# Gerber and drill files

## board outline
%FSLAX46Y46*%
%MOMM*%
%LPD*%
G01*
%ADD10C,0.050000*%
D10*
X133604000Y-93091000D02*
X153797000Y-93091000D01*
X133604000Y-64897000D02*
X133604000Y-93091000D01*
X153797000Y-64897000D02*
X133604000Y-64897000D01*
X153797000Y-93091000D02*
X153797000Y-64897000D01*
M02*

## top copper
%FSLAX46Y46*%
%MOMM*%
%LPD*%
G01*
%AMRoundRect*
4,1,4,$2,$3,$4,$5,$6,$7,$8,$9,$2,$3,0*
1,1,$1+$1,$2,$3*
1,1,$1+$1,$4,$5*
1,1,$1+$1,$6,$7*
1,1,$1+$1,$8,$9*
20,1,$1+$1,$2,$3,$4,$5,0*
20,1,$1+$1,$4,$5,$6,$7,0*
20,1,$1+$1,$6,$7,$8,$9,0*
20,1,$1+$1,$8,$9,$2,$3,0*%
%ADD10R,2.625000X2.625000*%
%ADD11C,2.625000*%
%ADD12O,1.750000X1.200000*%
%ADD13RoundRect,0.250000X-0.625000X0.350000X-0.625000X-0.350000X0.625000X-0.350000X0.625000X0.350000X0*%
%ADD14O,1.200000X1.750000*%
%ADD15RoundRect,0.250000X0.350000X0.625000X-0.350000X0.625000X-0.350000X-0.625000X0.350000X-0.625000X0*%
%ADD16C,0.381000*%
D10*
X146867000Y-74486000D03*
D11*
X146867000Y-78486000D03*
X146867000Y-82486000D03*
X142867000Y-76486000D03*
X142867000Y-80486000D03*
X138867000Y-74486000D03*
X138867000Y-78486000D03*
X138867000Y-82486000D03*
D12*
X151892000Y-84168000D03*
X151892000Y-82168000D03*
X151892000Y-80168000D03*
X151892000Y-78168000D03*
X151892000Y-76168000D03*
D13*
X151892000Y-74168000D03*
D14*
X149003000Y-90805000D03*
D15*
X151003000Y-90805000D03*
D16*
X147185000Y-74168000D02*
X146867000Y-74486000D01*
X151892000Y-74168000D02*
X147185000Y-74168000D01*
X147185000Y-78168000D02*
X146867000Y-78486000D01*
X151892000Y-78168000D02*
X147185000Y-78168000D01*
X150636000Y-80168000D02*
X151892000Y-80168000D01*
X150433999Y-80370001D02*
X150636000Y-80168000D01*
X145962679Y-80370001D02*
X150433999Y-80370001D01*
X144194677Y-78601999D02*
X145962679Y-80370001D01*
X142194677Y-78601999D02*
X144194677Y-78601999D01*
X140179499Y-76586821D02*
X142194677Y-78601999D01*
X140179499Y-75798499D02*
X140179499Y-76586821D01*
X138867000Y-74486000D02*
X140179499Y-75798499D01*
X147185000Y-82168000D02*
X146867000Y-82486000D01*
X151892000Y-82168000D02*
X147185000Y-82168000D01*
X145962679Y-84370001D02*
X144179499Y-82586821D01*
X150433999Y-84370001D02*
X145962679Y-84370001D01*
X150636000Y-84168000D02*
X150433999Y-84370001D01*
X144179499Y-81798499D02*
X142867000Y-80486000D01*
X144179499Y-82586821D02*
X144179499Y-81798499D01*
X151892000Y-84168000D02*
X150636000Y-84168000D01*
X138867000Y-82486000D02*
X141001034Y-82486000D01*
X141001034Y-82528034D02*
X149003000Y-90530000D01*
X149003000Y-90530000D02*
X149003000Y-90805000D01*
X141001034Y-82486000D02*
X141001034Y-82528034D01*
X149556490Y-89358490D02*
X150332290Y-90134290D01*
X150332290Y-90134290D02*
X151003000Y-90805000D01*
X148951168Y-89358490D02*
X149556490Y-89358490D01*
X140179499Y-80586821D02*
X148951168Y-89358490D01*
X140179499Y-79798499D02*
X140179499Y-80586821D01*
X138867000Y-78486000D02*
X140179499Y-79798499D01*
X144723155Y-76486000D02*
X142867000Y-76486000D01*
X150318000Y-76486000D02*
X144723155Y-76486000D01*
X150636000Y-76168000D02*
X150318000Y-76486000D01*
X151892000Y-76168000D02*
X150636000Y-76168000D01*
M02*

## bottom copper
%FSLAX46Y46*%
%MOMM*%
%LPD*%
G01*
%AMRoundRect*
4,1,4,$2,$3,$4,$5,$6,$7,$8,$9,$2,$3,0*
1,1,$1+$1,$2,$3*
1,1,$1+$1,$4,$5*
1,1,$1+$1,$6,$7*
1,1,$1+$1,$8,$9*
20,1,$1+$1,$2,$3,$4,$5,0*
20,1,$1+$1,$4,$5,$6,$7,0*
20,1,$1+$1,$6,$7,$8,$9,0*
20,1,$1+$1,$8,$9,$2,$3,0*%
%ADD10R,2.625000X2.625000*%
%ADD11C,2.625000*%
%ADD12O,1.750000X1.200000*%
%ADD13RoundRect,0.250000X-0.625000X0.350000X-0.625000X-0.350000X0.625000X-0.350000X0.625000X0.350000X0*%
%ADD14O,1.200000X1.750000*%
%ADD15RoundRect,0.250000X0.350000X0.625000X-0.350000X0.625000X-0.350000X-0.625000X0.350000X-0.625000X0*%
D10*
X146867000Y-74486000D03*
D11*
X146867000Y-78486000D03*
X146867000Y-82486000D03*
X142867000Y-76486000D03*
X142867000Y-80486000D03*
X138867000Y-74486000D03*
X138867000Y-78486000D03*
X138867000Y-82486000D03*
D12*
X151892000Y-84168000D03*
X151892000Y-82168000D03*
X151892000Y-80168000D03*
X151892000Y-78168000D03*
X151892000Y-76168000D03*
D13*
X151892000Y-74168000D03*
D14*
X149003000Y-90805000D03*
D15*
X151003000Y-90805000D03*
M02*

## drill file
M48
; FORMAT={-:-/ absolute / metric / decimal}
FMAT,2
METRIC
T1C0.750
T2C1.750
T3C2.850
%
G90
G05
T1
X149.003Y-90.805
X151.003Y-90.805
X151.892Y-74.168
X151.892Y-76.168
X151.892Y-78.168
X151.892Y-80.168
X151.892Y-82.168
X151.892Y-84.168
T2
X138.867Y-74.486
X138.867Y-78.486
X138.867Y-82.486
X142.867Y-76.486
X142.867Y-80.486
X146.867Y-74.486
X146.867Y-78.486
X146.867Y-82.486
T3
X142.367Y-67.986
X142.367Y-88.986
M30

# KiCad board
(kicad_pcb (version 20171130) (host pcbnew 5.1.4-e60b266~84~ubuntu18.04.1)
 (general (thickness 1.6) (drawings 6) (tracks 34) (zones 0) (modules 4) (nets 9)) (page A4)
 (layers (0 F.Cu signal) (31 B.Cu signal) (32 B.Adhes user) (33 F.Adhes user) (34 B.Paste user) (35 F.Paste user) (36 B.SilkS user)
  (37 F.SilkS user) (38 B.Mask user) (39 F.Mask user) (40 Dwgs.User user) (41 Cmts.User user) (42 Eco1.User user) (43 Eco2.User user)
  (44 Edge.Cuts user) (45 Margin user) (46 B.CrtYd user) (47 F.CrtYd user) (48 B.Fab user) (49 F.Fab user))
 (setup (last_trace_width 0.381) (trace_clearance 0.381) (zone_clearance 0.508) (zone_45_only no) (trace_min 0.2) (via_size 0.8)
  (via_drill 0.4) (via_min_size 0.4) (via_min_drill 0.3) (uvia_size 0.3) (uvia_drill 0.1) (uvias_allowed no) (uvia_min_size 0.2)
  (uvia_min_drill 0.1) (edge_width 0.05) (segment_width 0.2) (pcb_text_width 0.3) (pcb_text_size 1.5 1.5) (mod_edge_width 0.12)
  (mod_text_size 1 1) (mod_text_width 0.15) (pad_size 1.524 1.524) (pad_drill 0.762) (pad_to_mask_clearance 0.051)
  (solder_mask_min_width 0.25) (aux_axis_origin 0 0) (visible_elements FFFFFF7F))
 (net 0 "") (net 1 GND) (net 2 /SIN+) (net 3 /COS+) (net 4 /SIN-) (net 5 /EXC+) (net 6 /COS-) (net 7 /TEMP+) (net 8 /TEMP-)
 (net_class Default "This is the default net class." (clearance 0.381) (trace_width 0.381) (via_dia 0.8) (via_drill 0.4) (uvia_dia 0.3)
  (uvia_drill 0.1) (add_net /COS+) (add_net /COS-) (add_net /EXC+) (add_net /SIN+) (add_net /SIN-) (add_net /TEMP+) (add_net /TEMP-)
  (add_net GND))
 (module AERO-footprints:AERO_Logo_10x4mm (layer F.Cu) (at 148.844 67.056)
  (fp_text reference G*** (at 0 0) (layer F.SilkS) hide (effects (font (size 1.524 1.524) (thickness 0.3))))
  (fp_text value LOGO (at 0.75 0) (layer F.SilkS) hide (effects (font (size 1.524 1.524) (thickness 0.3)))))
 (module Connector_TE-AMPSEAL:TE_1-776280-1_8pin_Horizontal (layer F.Cu) (at 142.367 78.486 270)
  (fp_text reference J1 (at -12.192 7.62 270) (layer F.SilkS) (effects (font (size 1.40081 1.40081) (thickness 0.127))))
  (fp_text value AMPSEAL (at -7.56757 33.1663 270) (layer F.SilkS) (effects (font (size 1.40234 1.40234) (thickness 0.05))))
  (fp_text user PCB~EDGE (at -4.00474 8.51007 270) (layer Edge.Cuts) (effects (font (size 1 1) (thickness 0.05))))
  (pad 1 thru_hole rect (at -4 -4.5 270) (size 2.625 2.625) (drill 1.75) (layers *.Cu *.Mask) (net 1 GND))
  (pad 2 thru_hole circle (at 0 -4.5 270) (size 2.625 2.625) (drill 1.75) (layers *.Cu *.Mask) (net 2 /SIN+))
  (pad 3 thru_hole circle (at 4 -4.5 270) (size 2.625 2.625) (drill 1.75) (layers *.Cu *.Mask) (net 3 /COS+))
  (pad 4 thru_hole circle (at -2 -0.5 270) (size 2.625 2.625) (drill 1.75) (layers *.Cu *.Mask) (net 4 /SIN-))
  (pad 5 thru_hole circle (at 2 -0.5 270) (size 2.625 2.625) (drill 1.75) (layers *.Cu *.Mask) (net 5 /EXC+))
  (pad 6 thru_hole circle (at -4 3.5 270) (size 2.625 2.625) (drill 1.75) (layers *.Cu *.Mask) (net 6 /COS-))
  (pad 7 thru_hole circle (at 0 3.5 270) (size 2.625 2.625) (drill 1.75) (layers *.Cu *.Mask) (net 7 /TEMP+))
  (pad 8 thru_hole circle (at 4 3.5 270) (size 2.625 2.625) (drill 1.75) (layers *.Cu *.Mask) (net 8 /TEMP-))
  (pad Hole np_thru_hole circle (at -10.5 0 270) (size 2.85 2.85) (drill 2.85) (layers *.Cu *.Mask F.SilkS))
  (pad Hole np_thru_hole circle (at 10.5 0 270) (size 2.85 2.85) (drill 2.85) (layers *.Cu *.Mask F.SilkS)))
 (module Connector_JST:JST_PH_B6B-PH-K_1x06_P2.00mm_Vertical (layer F.Cu) (at 151.892 74.168 270)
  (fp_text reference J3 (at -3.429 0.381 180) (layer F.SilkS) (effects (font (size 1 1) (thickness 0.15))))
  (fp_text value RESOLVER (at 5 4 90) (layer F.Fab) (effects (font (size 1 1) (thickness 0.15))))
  (pad 6 thru_hole oval (at 10 0 270) (size 1.2 1.75) (drill 0.75) (layers *.Cu *.Mask) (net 5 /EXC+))
  (pad 5 thru_hole oval (at 8 0 270) (size 1.2 1.75) (drill 0.75) (layers *.Cu *.Mask) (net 3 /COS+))
  (pad 4 thru_hole oval (at 6 0 270) (size 1.2 1.75) (drill 0.75) (layers *.Cu *.Mask) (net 6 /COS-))
  (pad 3 thru_hole oval (at 4 0 270) (size 1.2 1.75) (drill 0.75) (layers *.Cu *.Mask) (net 2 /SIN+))
  (pad 2 thru_hole oval (at 2 0 270) (size 1.2 1.75) (drill 0.75) (layers *.Cu *.Mask) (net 4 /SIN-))
  (pad 1 thru_hole roundrect (at 0 0 270) (size 1.2 1.75) (drill 0.75) (layers *.Cu *.Mask) (roundrect_rratio 0.208333) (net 1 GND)))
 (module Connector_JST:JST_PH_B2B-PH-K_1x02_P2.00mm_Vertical (layer F.Cu) (at 151.003 90.805 180)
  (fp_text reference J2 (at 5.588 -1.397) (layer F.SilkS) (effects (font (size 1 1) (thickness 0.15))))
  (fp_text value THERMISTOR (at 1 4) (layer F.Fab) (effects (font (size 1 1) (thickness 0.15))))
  (pad 2 thru_hole oval (at 2 0 180) (size 1.2 1.75) (drill 0.75) (layers *.Cu *.Mask) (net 8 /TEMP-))
  (pad 1 thru_hole roundrect (at 0 0 180) (size 1.2 1.75) (drill 0.75) (layers *.Cu *.Mask) (roundrect_rratio 0.208333) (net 7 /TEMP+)))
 (gr_line (start 133.604 93.091) (end 153.797 93.091) (layer Edge.Cuts) (width 0.05))
 (gr_line (start 133.604 64.897) (end 133.604 93.091) (layer Edge.Cuts) (width 0.05))
 (gr_line (start 153.797 64.897) (end 133.604 64.897) (layer Edge.Cuts) (width 0.05))
 (gr_line (start 153.797 93.091) (end 153.797 64.897) (layer Edge.Cuts) (width 0.05))
 (segment (start 147.185 74.168) (end 146.867 74.486) (width 0.381) (layer F.Cu) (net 1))
 (segment (start 151.892 74.168) (end 147.185 74.168) (width 0.381) (layer F.Cu) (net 1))
 (segment (start 147.185 78.168) (end 146.867 78.486) (width 0.381) (layer F.Cu) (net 2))
 (segment (start 151.892 78.168) (end 147.185 78.168) (width 0.381) (layer F.Cu) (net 2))
 (segment (start 150.636 80.168) (end 151.892 80.168) (width 0.381) (layer F.Cu) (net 6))
 (segment (start 150.433999 80.370001) (end 150.636 80.168) (width 0.381) (layer F.Cu) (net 6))
 (segment (start 145.962679 80.370001) (end 150.433999 80.370001) (width 0.381) (layer F.Cu) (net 6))
 (segment (start 144.194677 78.601999) (end 145.962679 80.370001) (width 0.381) (layer F.Cu) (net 6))
 (segment (start 142.194677 78.601999) (end 144.194677 78.601999) (width 0.381) (layer F.Cu) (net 6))
 (segment (start 140.179499 76.586821) (end 142.194677 78.601999) (width 0.381) (layer F.Cu) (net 6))
 (segment (start 140.179499 75.798499) (end 140.179499 76.586821) (width 0.381) (layer F.Cu) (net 6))
 (segment (start 138.867 74.486) (end 140.179499 75.798499) (width 0.381) (layer F.Cu) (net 6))
 (segment (start 147.185 82.168) (end 146.867 82.486) (width 0.381) (layer F.Cu) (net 3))
 (segment (start 151.892 82.168) (end 147.185 82.168) (width 0.381) (layer F.Cu) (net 3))
 (segment (start 145.962679 84.370001) (end 144.179499 82.586821) (width 0.381) (layer F.Cu) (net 5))
 (segment (start 150.433999 84.370001) (end 145.962679 84.370001) (width 0.381) (layer F.Cu) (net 5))
 (segment (start 150.636 84.168) (end 150.433999 84.370001) (width 0.381) (layer F.Cu) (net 5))
 (segment (start 144.179499 81.798499) (end 142.867 80.486) (width 0.381) (layer F.Cu) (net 5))
 (segment (start 144.179499 82.586821) (end 144.179499 81.798499) (width 0.381) (layer F.Cu) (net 5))
 (segment (start 151.892 84.168) (end 150.636 84.168) (width 0.381) (layer F.Cu) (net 5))
 (segment (start 138.867 82.486) (end 141.001034 82.486) (width 0.381) (layer F.Cu) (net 8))
 (segment (start 141.001034 82.528034) (end 149.003 90.53) (width 0.381) (layer F.Cu) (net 8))
 (segment (start 149.003 90.53) (end 149.003 90.805) (width 0.381) (layer F.Cu) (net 8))
 (segment (start 141.001034 82.486) (end 141.001034 82.528034) (width 0.381) (layer F.Cu) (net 8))
 (segment (start 149.55649 89.35849) (end 150.33229 90.13429) (width 0.381) (layer F.Cu) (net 7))
 (segment (start 150.33229 90.13429) (end 151.003 90.805) (width 0.381) (layer F.Cu) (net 7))
 (segment (start 148.951168 89.35849) (end 149.55649 89.35849) (width 0.381) (layer F.Cu) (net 7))
 (segment (start 140.179499 80.586821) (end 148.951168 89.35849) (width 0.381) (layer F.Cu) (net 7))
 (segment (start 140.179499 79.798499) (end 140.179499 80.586821) (width 0.381) (layer F.Cu) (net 7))
 (segment (start 138.867 78.486) (end 140.179499 79.798499) (width 0.381) (layer F.Cu) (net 7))
 (segment (start 144.723155 76.486) (end 142.867 76.486) (width 0.381) (layer F.Cu) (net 4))
 (segment (start 150.318 76.486) (end 144.723155 76.486) (width 0.381) (layer F.Cu) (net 4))
 (segment (start 150.636 76.168) (end 150.318 76.486) (width 0.381) (layer F.Cu) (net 4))
 (segment (start 151.892 76.168) (end 150.636 76.168) (width 0.381) (layer F.Cu) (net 4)))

